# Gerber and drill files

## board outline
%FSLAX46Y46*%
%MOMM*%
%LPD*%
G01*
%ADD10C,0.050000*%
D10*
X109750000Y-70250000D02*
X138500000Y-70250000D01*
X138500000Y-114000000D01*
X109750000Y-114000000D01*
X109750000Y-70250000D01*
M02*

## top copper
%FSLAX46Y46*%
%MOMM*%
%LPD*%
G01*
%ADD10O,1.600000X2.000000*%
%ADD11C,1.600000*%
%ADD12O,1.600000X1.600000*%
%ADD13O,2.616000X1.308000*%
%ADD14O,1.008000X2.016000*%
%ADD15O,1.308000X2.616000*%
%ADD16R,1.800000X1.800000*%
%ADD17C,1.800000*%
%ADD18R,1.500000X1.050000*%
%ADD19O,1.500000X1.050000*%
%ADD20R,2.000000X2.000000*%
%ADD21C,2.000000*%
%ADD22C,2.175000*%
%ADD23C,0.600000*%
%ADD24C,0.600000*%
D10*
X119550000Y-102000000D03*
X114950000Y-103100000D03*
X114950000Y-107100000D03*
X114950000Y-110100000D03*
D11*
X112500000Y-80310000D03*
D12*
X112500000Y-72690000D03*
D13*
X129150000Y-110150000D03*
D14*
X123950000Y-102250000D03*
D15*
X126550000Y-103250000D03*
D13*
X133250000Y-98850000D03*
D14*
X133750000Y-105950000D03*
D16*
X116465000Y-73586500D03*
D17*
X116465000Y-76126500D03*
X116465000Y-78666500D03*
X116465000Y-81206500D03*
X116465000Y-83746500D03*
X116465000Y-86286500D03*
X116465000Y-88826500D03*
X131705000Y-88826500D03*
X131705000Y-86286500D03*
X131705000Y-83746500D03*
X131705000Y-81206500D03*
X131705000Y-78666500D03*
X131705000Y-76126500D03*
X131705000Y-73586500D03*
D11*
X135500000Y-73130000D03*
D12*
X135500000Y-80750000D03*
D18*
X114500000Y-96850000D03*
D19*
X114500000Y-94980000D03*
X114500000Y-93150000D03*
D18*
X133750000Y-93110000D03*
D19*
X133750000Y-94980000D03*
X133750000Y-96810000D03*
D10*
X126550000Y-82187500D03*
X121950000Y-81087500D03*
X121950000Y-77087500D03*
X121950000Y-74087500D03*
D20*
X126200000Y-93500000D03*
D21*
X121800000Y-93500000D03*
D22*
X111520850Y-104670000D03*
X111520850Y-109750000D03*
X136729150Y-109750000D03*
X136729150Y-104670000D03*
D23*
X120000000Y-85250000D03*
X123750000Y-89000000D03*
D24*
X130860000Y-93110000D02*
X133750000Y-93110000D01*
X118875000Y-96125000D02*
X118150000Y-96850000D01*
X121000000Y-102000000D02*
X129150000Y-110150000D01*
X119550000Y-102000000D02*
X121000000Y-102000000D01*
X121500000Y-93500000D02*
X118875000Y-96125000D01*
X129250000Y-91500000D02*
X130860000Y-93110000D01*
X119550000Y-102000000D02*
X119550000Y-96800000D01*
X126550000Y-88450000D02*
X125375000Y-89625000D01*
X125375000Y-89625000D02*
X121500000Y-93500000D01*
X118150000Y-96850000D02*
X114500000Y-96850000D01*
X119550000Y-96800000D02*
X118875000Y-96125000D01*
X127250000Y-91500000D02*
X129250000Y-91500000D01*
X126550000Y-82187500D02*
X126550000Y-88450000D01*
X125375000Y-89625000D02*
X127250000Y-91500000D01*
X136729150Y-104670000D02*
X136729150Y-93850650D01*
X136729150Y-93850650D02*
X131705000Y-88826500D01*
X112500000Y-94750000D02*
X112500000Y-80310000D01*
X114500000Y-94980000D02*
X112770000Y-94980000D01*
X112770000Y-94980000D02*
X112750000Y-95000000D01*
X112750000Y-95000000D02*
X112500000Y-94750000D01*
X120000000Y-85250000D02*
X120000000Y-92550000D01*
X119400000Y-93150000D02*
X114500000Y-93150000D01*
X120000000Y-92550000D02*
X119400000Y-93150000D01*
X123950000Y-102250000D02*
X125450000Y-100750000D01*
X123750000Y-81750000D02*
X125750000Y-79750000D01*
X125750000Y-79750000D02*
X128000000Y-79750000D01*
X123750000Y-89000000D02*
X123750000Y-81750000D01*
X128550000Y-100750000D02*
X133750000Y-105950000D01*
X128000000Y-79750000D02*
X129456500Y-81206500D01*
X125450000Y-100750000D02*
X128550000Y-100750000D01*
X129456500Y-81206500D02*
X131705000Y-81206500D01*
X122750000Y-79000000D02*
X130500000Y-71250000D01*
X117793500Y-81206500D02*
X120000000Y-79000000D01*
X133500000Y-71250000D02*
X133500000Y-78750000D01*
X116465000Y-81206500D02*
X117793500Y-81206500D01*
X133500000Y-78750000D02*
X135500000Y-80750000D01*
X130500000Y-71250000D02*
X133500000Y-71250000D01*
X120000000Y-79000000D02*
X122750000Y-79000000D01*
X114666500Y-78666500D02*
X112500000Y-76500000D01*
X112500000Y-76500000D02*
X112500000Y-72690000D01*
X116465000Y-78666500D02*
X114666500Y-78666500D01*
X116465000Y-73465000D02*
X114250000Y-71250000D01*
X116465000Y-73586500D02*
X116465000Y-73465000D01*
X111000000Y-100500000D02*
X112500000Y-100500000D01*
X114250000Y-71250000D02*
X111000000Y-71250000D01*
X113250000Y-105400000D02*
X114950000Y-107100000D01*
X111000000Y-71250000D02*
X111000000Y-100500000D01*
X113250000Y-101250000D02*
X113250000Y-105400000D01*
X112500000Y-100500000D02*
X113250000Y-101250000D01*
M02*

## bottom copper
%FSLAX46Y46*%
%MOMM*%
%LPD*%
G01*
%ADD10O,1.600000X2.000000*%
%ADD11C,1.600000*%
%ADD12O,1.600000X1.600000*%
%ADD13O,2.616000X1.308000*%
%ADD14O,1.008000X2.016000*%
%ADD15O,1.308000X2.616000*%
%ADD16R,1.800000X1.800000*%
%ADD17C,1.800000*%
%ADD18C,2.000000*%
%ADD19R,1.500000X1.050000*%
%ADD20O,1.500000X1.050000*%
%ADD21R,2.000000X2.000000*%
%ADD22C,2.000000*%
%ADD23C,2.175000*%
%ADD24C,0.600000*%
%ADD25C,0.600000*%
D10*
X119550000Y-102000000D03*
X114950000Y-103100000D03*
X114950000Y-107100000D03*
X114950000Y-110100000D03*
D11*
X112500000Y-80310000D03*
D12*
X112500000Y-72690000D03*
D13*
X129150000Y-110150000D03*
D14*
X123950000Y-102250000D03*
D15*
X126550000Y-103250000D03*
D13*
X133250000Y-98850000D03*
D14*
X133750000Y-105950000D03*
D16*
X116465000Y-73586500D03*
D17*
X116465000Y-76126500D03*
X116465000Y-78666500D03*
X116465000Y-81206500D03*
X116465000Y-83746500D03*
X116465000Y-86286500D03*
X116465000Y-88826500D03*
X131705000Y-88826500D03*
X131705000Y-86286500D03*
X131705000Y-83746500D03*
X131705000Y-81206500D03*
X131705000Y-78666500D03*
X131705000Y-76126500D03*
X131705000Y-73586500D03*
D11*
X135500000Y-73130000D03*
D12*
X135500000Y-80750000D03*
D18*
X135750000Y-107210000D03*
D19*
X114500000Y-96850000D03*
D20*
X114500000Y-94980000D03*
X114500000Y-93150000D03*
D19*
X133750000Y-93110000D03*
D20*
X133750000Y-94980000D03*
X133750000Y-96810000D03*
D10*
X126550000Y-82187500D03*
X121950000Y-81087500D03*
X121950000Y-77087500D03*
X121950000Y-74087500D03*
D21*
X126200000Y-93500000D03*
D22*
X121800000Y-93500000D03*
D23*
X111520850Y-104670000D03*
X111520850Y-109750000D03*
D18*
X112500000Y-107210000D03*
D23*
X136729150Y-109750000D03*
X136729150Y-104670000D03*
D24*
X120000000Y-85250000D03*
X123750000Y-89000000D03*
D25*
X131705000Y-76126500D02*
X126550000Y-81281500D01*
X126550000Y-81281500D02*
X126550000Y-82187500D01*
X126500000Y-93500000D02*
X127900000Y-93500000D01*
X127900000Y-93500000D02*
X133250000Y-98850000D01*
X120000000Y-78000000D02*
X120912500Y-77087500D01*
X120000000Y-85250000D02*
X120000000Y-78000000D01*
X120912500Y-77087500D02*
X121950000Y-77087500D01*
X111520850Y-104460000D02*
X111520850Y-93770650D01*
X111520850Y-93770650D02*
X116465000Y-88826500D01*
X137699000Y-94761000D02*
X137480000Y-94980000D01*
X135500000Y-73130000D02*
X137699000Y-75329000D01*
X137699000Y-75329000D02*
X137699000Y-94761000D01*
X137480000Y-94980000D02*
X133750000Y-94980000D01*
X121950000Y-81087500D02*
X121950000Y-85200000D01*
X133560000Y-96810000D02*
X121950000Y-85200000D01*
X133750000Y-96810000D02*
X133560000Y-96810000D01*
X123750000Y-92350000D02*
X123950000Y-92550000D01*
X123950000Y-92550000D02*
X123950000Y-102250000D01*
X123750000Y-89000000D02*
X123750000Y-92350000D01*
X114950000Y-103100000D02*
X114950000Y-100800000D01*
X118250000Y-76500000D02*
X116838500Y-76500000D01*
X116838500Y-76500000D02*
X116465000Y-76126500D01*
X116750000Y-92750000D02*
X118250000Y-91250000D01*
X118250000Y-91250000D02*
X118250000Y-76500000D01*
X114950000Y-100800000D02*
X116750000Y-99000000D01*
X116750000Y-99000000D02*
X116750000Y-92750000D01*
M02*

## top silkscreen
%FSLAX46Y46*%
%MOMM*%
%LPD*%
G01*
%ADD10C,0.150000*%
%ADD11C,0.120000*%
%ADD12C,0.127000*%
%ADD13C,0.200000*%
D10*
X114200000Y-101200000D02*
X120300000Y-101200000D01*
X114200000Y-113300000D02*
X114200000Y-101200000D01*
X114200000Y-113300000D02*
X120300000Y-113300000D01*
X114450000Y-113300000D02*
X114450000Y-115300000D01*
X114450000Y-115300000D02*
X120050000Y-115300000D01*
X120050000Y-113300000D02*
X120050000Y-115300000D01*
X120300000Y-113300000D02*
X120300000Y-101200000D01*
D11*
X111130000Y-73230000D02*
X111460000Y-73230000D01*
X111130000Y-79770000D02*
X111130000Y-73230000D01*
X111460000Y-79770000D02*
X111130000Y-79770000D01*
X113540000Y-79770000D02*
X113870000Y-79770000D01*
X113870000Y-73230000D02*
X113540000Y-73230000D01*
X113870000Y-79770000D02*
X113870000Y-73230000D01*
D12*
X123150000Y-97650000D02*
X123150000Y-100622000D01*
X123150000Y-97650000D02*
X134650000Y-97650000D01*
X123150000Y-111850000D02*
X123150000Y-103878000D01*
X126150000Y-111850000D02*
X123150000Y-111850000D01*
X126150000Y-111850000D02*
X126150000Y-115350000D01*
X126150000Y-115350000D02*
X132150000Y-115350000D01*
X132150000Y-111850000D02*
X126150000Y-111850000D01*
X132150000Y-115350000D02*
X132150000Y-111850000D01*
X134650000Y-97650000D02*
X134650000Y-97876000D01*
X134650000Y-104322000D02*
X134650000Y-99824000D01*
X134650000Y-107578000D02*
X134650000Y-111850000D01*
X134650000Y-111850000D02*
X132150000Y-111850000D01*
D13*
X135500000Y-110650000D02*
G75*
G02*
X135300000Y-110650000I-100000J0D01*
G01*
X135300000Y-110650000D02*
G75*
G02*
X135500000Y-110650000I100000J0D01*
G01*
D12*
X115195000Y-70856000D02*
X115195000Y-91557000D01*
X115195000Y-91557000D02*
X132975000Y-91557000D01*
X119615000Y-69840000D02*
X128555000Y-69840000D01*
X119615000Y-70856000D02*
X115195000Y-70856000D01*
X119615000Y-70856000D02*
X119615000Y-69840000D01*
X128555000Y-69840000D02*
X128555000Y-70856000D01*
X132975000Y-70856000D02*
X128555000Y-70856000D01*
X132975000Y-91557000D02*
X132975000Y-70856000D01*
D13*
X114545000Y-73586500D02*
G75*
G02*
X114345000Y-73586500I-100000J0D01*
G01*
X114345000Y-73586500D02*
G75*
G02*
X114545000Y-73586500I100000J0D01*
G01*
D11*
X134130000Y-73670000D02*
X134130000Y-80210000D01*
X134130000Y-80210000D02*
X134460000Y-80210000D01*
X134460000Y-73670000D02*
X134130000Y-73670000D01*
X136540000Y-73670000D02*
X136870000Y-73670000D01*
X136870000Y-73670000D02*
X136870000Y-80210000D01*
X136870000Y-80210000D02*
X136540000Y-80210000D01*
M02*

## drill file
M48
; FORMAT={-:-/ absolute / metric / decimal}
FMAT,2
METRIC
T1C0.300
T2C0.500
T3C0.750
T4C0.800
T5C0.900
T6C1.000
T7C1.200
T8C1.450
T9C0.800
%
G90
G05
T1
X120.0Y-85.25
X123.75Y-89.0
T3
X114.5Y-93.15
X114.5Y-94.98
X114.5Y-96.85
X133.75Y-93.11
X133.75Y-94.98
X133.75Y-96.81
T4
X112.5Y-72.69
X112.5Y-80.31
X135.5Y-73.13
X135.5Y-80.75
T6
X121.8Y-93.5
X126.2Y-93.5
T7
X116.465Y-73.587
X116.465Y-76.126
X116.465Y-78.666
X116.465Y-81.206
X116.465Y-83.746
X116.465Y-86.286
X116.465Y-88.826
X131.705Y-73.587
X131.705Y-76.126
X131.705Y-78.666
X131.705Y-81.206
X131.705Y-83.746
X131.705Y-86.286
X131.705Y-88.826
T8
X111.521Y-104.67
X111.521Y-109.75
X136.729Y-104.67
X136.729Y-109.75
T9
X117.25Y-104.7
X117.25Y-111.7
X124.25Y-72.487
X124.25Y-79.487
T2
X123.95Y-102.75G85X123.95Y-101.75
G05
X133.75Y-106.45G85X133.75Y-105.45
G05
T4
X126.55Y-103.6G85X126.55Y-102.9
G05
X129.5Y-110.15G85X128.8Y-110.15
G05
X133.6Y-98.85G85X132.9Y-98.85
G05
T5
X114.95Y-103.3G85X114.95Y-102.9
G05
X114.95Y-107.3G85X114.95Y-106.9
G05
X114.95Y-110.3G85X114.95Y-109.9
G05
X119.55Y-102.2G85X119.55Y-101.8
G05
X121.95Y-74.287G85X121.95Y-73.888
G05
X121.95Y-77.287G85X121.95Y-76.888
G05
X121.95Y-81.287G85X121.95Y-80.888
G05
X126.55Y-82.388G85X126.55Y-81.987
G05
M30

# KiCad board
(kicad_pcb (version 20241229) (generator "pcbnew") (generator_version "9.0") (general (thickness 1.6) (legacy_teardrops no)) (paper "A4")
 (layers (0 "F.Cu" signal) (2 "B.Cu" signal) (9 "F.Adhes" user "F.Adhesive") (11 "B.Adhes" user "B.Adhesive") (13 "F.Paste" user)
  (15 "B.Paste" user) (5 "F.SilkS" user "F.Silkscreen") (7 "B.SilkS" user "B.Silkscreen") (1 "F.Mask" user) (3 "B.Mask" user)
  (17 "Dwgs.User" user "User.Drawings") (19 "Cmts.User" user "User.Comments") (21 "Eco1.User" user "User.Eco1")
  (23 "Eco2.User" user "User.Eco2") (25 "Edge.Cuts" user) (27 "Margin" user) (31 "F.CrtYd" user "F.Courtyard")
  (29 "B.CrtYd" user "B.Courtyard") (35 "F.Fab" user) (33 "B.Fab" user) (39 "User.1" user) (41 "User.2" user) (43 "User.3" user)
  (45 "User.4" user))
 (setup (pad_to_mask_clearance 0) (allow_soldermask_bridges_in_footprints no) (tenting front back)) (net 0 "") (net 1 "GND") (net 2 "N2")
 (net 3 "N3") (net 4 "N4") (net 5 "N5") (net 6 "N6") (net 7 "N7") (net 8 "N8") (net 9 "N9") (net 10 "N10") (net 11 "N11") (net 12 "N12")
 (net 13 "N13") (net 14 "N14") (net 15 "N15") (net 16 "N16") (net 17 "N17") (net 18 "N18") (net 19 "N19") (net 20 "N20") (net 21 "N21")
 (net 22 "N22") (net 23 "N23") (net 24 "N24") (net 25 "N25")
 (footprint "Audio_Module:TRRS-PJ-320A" (layer "F.Cu") (at 117.25 113.3 180)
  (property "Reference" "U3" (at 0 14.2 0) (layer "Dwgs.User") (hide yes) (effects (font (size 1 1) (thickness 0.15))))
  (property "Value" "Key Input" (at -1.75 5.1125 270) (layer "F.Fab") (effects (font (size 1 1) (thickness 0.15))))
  (fp_line (start 3.05 12.1) (end -3.05 12.1) (stroke (width 0.15) (type solid)) (layer "F.SilkS"))
  (fp_line (start 3.05 0) (end 3.05 12.1) (stroke (width 0.15) (type solid)) (layer "F.SilkS"))
  (fp_line (start 3.05 0) (end -3.05 0) (stroke (width 0.15) (type solid)) (layer "F.SilkS"))
  (fp_line (start 2.8 0) (end 2.8 -2) (stroke (width 0.15) (type solid)) (layer "F.SilkS"))
  (fp_line (start 2.8 -2) (end -2.8 -2) (stroke (width 0.15) (type solid)) (layer "F.SilkS"))
  (fp_line (start -2.8 0) (end -2.8 -2) (stroke (width 0.15) (type solid)) (layer "F.SilkS"))
  (fp_line (start -3.05 0) (end -3.05 12.1) (stroke (width 0.15) (type solid)) (layer "F.SilkS"))
  (pad "" np_thru_hole circle (at 0 1.6 180) (size 0.8 0.8) (drill 0.8) (layers "*.Cu" "*.Mask"))
  (pad "" np_thru_hole circle (at 0 8.6 180) (size 0.8 0.8) (drill 0.8) (layers "*.Cu" "*.Mask"))
  (pad "1" thru_hole oval (at -2.3 11.3 180) (size 1.6 2) (drill oval 0.9 1.3) (layers "*.Cu" "*.Mask") (remove_unused_layers no)
   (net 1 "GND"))
  (pad "2" thru_hole oval (at 2.3 10.2 180) (size 1.6 2) (drill oval 0.9 1.3) (layers "*.Cu" "*.Mask") (remove_unused_layers no)
   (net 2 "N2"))
  (pad "3" thru_hole oval (at 2.3 6.2 180) (size 1.6 2) (drill oval 0.9 1.3) (layers "*.Cu" "*.Mask") (remove_unused_layers no) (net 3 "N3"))
  (pad "4" thru_hole oval (at 2.3 3.2 180) (size 1.6 2) (drill oval 0.9 1.3) (layers "*.Cu" "*.Mask") (remove_unused_layers no) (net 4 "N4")))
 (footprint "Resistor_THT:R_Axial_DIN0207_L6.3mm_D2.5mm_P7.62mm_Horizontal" (layer "F.Cu") (at 112.5 80.31 90)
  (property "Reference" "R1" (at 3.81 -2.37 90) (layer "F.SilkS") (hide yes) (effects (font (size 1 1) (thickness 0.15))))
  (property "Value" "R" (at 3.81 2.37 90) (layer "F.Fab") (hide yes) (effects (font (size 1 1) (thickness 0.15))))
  (fp_line (start 7.08 -1.37) (end 7.08 -1.04) (stroke (width 0.12) (type solid)) (layer "F.SilkS"))
  (fp_line (start 0.54 -1.37) (end 7.08 -1.37) (stroke (width 0.12) (type solid)) (layer "F.SilkS"))
  (fp_line (start 0.54 -1.04) (end 0.54 -1.37) (stroke (width 0.12) (type solid)) (layer "F.SilkS"))
  (fp_line (start 0.54 1.04) (end 0.54 1.37) (stroke (width 0.12) (type solid)) (layer "F.SilkS"))
  (fp_line (start 7.08 1.37) (end 7.08 1.04) (stroke (width 0.12) (type solid)) (layer "F.SilkS"))
  (fp_line (start 0.54 1.37) (end 7.08 1.37) (stroke (width 0.12) (type solid)) (layer "F.SilkS"))
  (pad "1" thru_hole circle (at 0 0 90) (size 1.6 1.6) (drill 0.8) (layers "*.Cu" "*.Mask") (remove_unused_layers no) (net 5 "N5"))
  (pad "2" thru_hole oval (at 7.62 0 90) (size 1.6 1.6) (drill 0.8) (layers "*.Cu" "*.Mask") (remove_unused_layers no) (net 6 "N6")))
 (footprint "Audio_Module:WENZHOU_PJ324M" (layer "F.Cu") (at 129.15 104.75 180)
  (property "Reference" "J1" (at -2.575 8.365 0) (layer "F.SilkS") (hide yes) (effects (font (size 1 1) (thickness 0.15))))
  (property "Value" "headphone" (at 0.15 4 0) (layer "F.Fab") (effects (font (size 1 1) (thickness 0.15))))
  (fp_line (start 6 7.1) (end 6 4.128) (stroke (width 0.127) (type solid)) (layer "F.SilkS"))
  (fp_line (start 6 7.1) (end -5.5 7.1) (stroke (width 0.127) (type solid)) (layer "F.SilkS"))
  (fp_line (start 6 -7.1) (end 6 0.872) (stroke (width 0.127) (type solid)) (layer "F.SilkS"))
  (fp_line (start 3 -7.1) (end 6 -7.1) (stroke (width 0.127) (type solid)) (layer "F.SilkS"))
  (fp_line (start 3 -7.1) (end 3 -10.6) (stroke (width 0.127) (type solid)) (layer "F.SilkS"))
  (fp_line (start 3 -10.6) (end -3 -10.6) (stroke (width 0.127) (type solid)) (layer "F.SilkS"))
  (fp_line (start -3 -7.1) (end 3 -7.1) (stroke (width 0.127) (type solid)) (layer "F.SilkS"))
  (fp_line (start -3 -10.6) (end -3 -7.1) (stroke (width 0.127) (type solid)) (layer "F.SilkS"))
  (fp_line (start -5.5 7.1) (end -5.5 6.874) (stroke (width 0.127) (type solid)) (layer "F.SilkS"))
  (fp_line (start -5.5 0.428) (end -5.5 4.926) (stroke (width 0.127) (type solid)) (layer "F.SilkS"))
  (fp_line (start -5.5 -2.828) (end -5.5 -7.1) (stroke (width 0.127) (type solid)) (layer "F.SilkS"))
  (fp_line (start -5.5 -7.1) (end -3 -7.1) (stroke (width 0.127) (type solid)) (layer "F.SilkS"))
  (fp_circle (center -6.25 -5.9) (end -6.15 -5.9) (stroke (width 0.2) (type solid)) (fill no) (layer "F.SilkS"))
  (pad "1" thru_hole oval (at 0 -5.4 180) (size 2.616 1.308) (drill oval 1.5 0.8) (layers "*.Cu" "*.Mask") (remove_unused_layers no)
   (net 1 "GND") (solder_mask_margin 0.102))
  (pad "2" thru_hole oval (at 5.2 2.5 180) (size 1.008 2.016) (drill oval 0.5 1.5) (layers "*.Cu" "*.Mask") (remove_unused_layers no)
   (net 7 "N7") (solder_mask_margin 0.102))
  (pad "3" thru_hole oval (at 2.6 1.5 180) (size 1.308 2.616) (drill oval 0.8 1.5) (layers "*.Cu" "*.Mask") (remove_unused_layers no)
   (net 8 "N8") (solder_mask_margin 0.102))
  (pad "4" thru_hole oval (at -4.1 5.9 180) (size 2.616 1.308) (drill oval 1.5 0.8) (layers "*.Cu" "*.Mask") (remove_unused_layers no)
   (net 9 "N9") (solder_mask_margin 0.102))
  (pad "5" thru_hole oval (at -4.6 -1.2 180) (size 1.008 2.016) (drill oval 0.5 1.5) (layers "*.Cu" "*.Mask") (remove_unused_layers no)
   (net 7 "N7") (solder_mask_margin 0.102)))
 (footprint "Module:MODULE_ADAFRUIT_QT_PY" (layer "F.Cu") (at 124.085 81.2065)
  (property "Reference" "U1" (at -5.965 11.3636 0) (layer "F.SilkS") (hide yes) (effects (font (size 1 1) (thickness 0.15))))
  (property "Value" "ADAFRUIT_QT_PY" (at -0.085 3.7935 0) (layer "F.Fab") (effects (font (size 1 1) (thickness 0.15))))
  (fp_line (start -8.89 -10.3505) (end -8.89 10.3505) (stroke (width 0.127) (type solid)) (layer "F.SilkS"))
  (fp_line (start -8.89 10.3505) (end 8.89 10.3505) (stroke (width 0.127) (type solid)) (layer "F.SilkS"))
  (fp_line (start -4.47 -11.3665) (end 4.47 -11.3665) (stroke (width 0.127) (type solid)) (layer "F.SilkS"))
  (fp_line (start -4.47 -10.3505) (end -8.89 -10.3505) (stroke (width 0.127) (type solid)) (layer "F.SilkS"))
  (fp_line (start -4.47 -10.3505) (end -4.47 -11.3665) (stroke (width 0.127) (type solid)) (layer "F.SilkS"))
  (fp_line (start 4.47 -11.3665) (end 4.47 -10.3505) (stroke (width 0.127) (type solid)) (layer "F.SilkS"))
  (fp_line (start 8.89 -10.3505) (end 4.47 -10.3505) (stroke (width 0.127) (type solid)) (layer "F.SilkS"))
  (fp_line (start 8.89 10.3505) (end 8.89 -10.3505) (stroke (width 0.127) (type solid)) (layer "F.SilkS"))
  (fp_circle (center -9.64 -7.62) (end -9.54 -7.62) (stroke (width 0.2) (type solid)) (fill no) (layer "F.SilkS"))
  (pad "1" thru_hole rect (at -7.62 -7.62) (size 1.8 1.8) (drill 1.2) (layers "*.Cu" "*.Mask") (remove_unused_layers no) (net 3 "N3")
   (solder_mask_margin 0.102))
  (pad "2" thru_hole circle (at -7.62 -5.08) (size 1.8 1.8) (drill 1.2) (layers "*.Cu" "*.Mask") (remove_unused_layers no) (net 2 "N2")
   (solder_mask_margin 0.102))
  (pad "3" thru_hole circle (at -7.62 -2.54) (size 1.8 1.8) (drill 1.2) (layers "*.Cu" "*.Mask") (remove_unused_layers no) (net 6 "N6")
   (solder_mask_margin 0.102))
  (pad "4" thru_hole circle (at -7.62 0) (size 1.8 1.8) (drill 1.2) (layers "*.Cu" "*.Mask") (remove_unused_layers no) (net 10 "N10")
   (solder_mask_margin 0.102))
  (pad "5" thru_hole circle (at -7.62 2.54) (size 1.8 1.8) (drill 1.2) (layers "*.Cu" "*.Mask") (remove_unused_layers no) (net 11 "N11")
   (solder_mask_margin 0.102))
  (pad "6" thru_hole circle (at -7.62 5.08) (size 1.8 1.8) (drill 1.2) (layers "*.Cu" "*.Mask") (remove_unused_layers no) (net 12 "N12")
   (solder_mask_margin 0.102))
  (pad "7" thru_hole circle (at -7.62 7.62) (size 1.8 1.8) (drill 1.2) (layers "*.Cu" "*.Mask") (remove_unused_layers no) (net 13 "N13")
   (solder_mask_margin 0.102))
  (pad "8" thru_hole circle (at 7.62 7.62) (size 1.8 1.8) (drill 1.2) (layers "*.Cu" "*.Mask") (remove_unused_layers no) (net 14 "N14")
   (solder_mask_margin 0.102))
  (pad "9" thru_hole circle (at 7.62 5.08) (size 1.8 1.8) (drill 1.2) (layers "*.Cu" "*.Mask") (remove_unused_layers no) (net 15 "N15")
   (solder_mask_margin 0.102))
  (pad "10" thru_hole circle (at 7.62 2.54) (size 1.8 1.8) (drill 1.2) (layers "*.Cu" "*.Mask") (remove_unused_layers no) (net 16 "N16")
   (solder_mask_margin 0.102))
  (pad "11" thru_hole circle (at 7.62 0) (size 1.8 1.8) (drill 1.2) (layers "*.Cu" "*.Mask") (remove_unused_layers no) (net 7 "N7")
   (solder_mask_margin 0.102))
  (pad "12" thru_hole circle (at 7.62 -2.54) (size 1.8 1.8) (drill 1.2) (layers "*.Cu" "*.Mask") (remove_unused_layers no) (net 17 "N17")
   (solder_mask_margin 0.102))
  (pad "13" thru_hole circle (at 7.62 -5.08) (size 1.8 1.8) (drill 1.2) (layers "*.Cu" "*.Mask") (remove_unused_layers no) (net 1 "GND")
   (solder_mask_margin 0.102))
  (pad "14" thru_hole circle (at 7.62 -7.62) (size 1.8 1.8) (drill 1.2) (layers "*.Cu" "*.Mask") (remove_unused_layers no) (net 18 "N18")
   (solder_mask_margin 0.102)))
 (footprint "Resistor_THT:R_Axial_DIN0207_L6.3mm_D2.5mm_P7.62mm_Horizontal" (layer "F.Cu") (at 135.5 73.13 -90)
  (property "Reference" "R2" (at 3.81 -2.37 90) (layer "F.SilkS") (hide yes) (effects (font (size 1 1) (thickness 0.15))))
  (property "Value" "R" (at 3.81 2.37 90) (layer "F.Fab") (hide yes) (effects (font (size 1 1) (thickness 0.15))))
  (fp_line (start 0.54 1.37) (end 7.08 1.37) (stroke (width 0.12) (type solid)) (layer "F.SilkS"))
  (fp_line (start 7.08 1.37) (end 7.08 1.04) (stroke (width 0.12) (type solid)) (layer "F.SilkS"))
  (fp_line (start 0.54 1.04) (end 0.54 1.37) (stroke (width 0.12) (type solid)) (layer "F.SilkS"))
  (fp_line (start 0.54 -1.04) (end 0.54 -1.37) (stroke (width 0.12) (type solid)) (layer "F.SilkS"))
  (fp_line (start 0.54 -1.37) (end 7.08 -1.37) (stroke (width 0.12) (type solid)) (layer "F.SilkS"))
  (fp_line (start 7.08 -1.37) (end 7.08 -1.04) (stroke (width 0.12) (type solid)) (layer "F.SilkS"))
  (pad "1" thru_hole circle (at 0 0 270) (size 1.6 1.6) (drill 0.8) (layers "*.Cu" "*.Mask") (remove_unused_layers no) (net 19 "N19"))
  (pad "2" thru_hole oval (at 7.62 0 270) (size 1.6 1.6) (drill 0.8) (layers "*.Cu" "*.Mask") (remove_unused_layers no) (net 10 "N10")))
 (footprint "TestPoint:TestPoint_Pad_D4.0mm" (layer "B.Cu") (at 135.75 107.21 180)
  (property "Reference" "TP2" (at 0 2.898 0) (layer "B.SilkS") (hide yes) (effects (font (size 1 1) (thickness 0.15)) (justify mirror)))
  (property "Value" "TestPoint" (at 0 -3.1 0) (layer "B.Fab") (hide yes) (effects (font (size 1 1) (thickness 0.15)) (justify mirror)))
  (pad "1" smd circle (at 0 0 180) (size 2 2) (layers "B.Cu" "B.Mask") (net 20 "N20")))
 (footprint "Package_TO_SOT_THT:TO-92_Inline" (layer "B.Cu") (at 114.5 96.25 90)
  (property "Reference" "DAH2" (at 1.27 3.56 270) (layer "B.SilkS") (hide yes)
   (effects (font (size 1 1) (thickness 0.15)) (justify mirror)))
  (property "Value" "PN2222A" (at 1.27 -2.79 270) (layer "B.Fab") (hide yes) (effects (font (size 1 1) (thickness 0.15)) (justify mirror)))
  (pad "1" thru_hole rect (at -0.6 0 90) (size 1.05 1.5) (drill 0.75) (layers "*.Cu" "*.Mask") (remove_unused_layers no) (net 1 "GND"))
  (pad "2" thru_hole oval (at 1.27 0 90) (size 1.05 1.5) (drill 0.75) (layers "*.Cu" "*.Mask") (remove_unused_layers no) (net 5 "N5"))
  (pad "3" thru_hole oval (at 3.1 0 90) (size 1.05 1.5) (drill 0.75) (layers "*.Cu" "*.Mask") (remove_unused_layers no) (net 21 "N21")))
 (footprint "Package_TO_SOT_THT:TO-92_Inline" (layer "B.Cu") (at 133.75 93.71 -90)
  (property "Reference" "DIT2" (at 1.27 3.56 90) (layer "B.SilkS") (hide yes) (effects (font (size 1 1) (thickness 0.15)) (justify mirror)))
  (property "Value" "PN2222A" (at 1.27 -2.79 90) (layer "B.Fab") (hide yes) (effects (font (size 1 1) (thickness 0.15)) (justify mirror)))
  (pad "1" thru_hole rect (at -0.6 0 270) (size 1.05 1.5) (drill 0.75) (layers "*.Cu" "*.Mask") (remove_unused_layers no) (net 1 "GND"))
  (pad "2" thru_hole oval (at 1.27 0 270) (size 1.05 1.5) (drill 0.75) (layers "*.Cu" "*.Mask") (remove_unused_layers no) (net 19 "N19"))
  (pad "3" thru_hole oval (at 3.1 0 270) (size 1.05 1.5) (drill 0.75) (layers "*.Cu" "*.Mask") (remove_unused_layers no) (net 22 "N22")))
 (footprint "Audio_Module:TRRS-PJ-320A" (layer "B.Cu") (at 124.25 70.8875 180)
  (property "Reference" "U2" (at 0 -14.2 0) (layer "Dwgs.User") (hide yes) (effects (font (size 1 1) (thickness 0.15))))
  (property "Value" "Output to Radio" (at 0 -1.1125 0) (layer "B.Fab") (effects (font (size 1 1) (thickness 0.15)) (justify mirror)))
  (pad "" np_thru_hole circle (at 0 -8.6 180) (size 0.8 0.8) (drill 0.8) (layers "*.Cu" "*.Mask"))
  (pad "" np_thru_hole circle (at 0 -1.6 180) (size 0.8 0.8) (drill 0.8) (layers "*.Cu" "*.Mask"))
  (pad "1" thru_hole oval (at -2.3 -11.3 180) (size 1.6 2) (drill oval 0.9 1.3) (layers "*.Cu" "*.Mask") (remove_unused_layers no)
   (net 1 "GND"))
  (pad "2" thru_hole oval (at 2.3 -10.2 180) (size 1.6 2) (drill oval 0.9 1.3) (layers "*.Cu" "*.Mask") (remove_unused_layers no)
   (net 22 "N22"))
  (pad "3" thru_hole oval (at 2.3 -6.2 180) (size 1.6 2) (drill oval 0.9 1.3) (layers "*.Cu" "*.Mask") (remove_unused_layers no)
   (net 21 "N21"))
  (pad "4" thru_hole oval (at 2.3 -3.2 180) (size 1.6 2) (drill oval 0.9 1.3) (layers "*.Cu" "*.Mask") (remove_unused_layers no)
   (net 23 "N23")))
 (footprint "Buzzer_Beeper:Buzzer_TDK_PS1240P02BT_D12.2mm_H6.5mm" (layer "B.Cu") (at 126.5 93.5 180)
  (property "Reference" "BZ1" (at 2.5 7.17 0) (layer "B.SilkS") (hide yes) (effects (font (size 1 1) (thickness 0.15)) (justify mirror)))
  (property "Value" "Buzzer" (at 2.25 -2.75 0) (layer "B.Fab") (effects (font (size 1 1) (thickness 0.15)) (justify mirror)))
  (pad "1" thru_hole rect (at 0.3 0 180) (size 2 2) (drill 1) (layers "*.Cu" "*.Mask") (remove_unused_layers no) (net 9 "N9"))
  (pad "2" thru_hole circle (at 4.7 0 180) (size 2 2) (drill 1) (layers "*.Cu" "*.Mask") (remove_unused_layers no) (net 1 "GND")))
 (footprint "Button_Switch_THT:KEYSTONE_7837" (layer "B.Cu") (at 111.52085 107.21 -90)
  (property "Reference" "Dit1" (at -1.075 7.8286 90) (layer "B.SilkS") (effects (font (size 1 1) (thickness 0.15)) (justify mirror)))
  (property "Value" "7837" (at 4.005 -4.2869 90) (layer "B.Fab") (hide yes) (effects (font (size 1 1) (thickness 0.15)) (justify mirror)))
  (pad "1_1" thru_hole circle (at -2.54 0 270) (size 2.175 2.175) (drill 1.45) (layers "*.Cu" "*.Mask") (remove_unused_layers no)
   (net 13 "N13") (solder_mask_margin 0.102))
  (pad "1_2" thru_hole circle (at 2.54 0 270) (size 2.175 2.175) (drill 1.45) (layers "*.Cu" "*.Mask") (remove_unused_layers no)
   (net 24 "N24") (solder_mask_margin 0.102)))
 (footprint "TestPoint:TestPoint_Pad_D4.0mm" (layer "B.Cu") (at 112.5 107.21 180)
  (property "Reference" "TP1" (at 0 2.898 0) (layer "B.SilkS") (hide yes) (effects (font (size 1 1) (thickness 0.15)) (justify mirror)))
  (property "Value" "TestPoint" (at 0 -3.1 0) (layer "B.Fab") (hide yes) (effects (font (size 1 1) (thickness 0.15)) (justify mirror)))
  (pad "1" smd circle (at 0 0 180) (size 2 2) (layers "B.Cu" "B.Mask") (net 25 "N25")))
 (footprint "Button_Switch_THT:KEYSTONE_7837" (layer "B.Cu") (at 136.72915 107.21 90)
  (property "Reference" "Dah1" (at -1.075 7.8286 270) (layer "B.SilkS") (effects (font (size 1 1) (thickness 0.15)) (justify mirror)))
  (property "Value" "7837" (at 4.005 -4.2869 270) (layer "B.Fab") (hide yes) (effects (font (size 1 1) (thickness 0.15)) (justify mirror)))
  (pad "1_1" thru_hole circle (at -2.54 0 90) (size 2.175 2.175) (drill 1.45) (layers "*.Cu" "*.Mask") (remove_unused_layers no)
   (solder_mask_margin 0.102))
  (pad "1_2" thru_hole circle (at 2.54 0 90) (size 2.175 2.175) (drill 1.45) (layers "*.Cu" "*.Mask") (remove_unused_layers no)
   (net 14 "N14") (solder_mask_margin 0.102)))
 (gr_rect (start 109.75 70.25) (end 138.5 114) (stroke (width 0.05) (type default)) (fill no) (layer "Edge.Cuts"))
 (segment (start 130.86 93.11) (end 133.75 93.11) (width 0.6) (layer "F.Cu") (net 1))
 (segment (start 118.875 96.125) (end 118.15 96.85) (width 0.6) (layer "F.Cu") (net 1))
 (segment (start 121 102) (end 129.15 110.15) (width 0.6) (layer "F.Cu") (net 1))
 (segment (start 119.55 102) (end 121 102) (width 0.6) (layer "F.Cu") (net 1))
 (segment (start 121.5 93.5) (end 118.875 96.125) (width 0.6) (layer "F.Cu") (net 1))
 (segment (start 129.25 91.5) (end 130.86 93.11) (width 0.6) (layer "F.Cu") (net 1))
 (segment (start 119.55 102) (end 119.55 96.8) (width 0.6) (layer "F.Cu") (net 1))
 (segment (start 126.55 88.45) (end 125.375 89.625) (width 0.6) (layer "F.Cu") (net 1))
 (segment (start 125.375 89.625) (end 121.5 93.5) (width 0.6) (layer "F.Cu") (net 1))
 (segment (start 118.15 96.85) (end 114.5 96.85) (width 0.6) (layer "F.Cu") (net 1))
 (segment (start 119.55 96.8) (end 118.875 96.125) (width 0.6) (layer "F.Cu") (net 1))
 (segment (start 127.25 91.5) (end 129.25 91.5) (width 0.6) (layer "F.Cu") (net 1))
 (segment (start 126.55 82.1875) (end 126.55 88.45) (width 0.6) (layer "F.Cu") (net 1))
 (segment (start 125.375 89.625) (end 127.25 91.5) (width 0.6) (layer "F.Cu") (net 1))
 (segment (start 131.705 76.1265) (end 126.55 81.2815) (width 0.6) (layer "B.Cu") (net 1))
 (segment (start 126.55 81.2815) (end 126.55 82.1875) (width 0.6) (layer "B.Cu") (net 1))
 (segment (start 126.5 93.5) (end 127.9 93.5) (width 0.6) (layer "B.Cu") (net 9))
 (segment (start 127.9 93.5) (end 133.25 98.85) (width 0.6) (layer "B.Cu") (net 9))
 (segment (start 136.72915 104.67) (end 136.72915 93.85065) (width 0.6) (layer "F.Cu") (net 14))
 (segment (start 136.72915 93.85065) (end 131.705 88.8265) (width 0.6) (layer "F.Cu") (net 14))
 (segment (start 112.5 94.75) (end 112.5 80.31) (width 0.6) (layer "F.Cu") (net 5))
 (segment (start 114.5 94.98) (end 112.77 94.98) (width 0.6) (layer "F.Cu") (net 5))
 (segment (start 112.77 94.98) (end 112.75 95) (width 0.6) (layer "F.Cu") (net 5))
 (segment (start 112.75 95) (end 112.5 94.75) (width 0.6) (layer "F.Cu") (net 5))
 (segment (start 120 85.25) (end 120 92.55) (width 0.6) (layer "F.Cu") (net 21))
 (segment (start 119.4 93.15) (end 114.5 93.15) (width 0.6) (layer "F.Cu") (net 21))
 (segment (start 120 92.55) (end 119.4 93.15) (width 0.6) (layer "F.Cu") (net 21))
 (via (at 120 85.25) (size 0.6) (drill 0.3) (layers "F.Cu" "B.Cu") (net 21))
 (segment (start 120 78) (end 120.9125 77.0875) (width 0.6) (layer "B.Cu") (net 21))
 (segment (start 120 85.25) (end 120 78) (width 0.6) (layer "B.Cu") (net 21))
 (segment (start 120.9125 77.0875) (end 121.95 77.0875) (width 0.6) (layer "B.Cu") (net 21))
 (segment (start 111.52085 104.46) (end 111.52085 93.77065) (width 0.6) (layer "B.Cu") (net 13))
 (segment (start 111.52085 93.77065) (end 116.465 88.8265) (width 0.6) (layer "B.Cu") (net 13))
 (segment (start 137.699 94.761) (end 137.48 94.98) (width 0.6) (layer "B.Cu") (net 19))
 (segment (start 135.5 73.13) (end 137.699 75.329) (width 0.6) (layer "B.Cu") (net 19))
 (segment (start 137.699 75.329) (end 137.699 94.761) (width 0.6) (layer "B.Cu") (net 19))
 (segment (start 137.48 94.98) (end 133.75 94.98) (width 0.6) (layer "B.Cu") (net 19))
 (segment (start 121.95 81.0875) (end 121.95 85.2) (width 0.6) (layer "B.Cu") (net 22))
 (segment (start 133.56 96.81) (end 121.95 85.2) (width 0.6) (layer "B.Cu") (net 22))
 (segment (start 133.75 96.81) (end 133.56 96.81) (width 0.6) (layer "B.Cu") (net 22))
 (segment (start 123.95 102.25) (end 125.45 100.75) (width 0.6) (layer "F.Cu") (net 7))
 (segment (start 123.75 81.75) (end 125.75 79.75) (width 0.6) (layer "F.Cu") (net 7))
 (segment (start 125.75 79.75) (end 128 79.75) (width 0.6) (layer "F.Cu") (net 7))
 (segment (start 123.75 89) (end 123.75 81.75) (width 0.6) (layer "F.Cu") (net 7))
 (segment (start 128.55 100.75) (end 133.75 105.95) (width 0.6) (layer "F.Cu") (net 7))
 (segment (start 128 79.75) (end 129.4565 81.2065) (width 0.6) (layer "F.Cu") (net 7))
 (segment (start 125.45 100.75) (end 128.55 100.75) (width 0.6) (layer "F.Cu") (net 7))
 (segment (start 129.4565 81.2065) (end 131.705 81.2065) (width 0.6) (layer "F.Cu") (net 7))
 (via (at 123.75 89) (size 0.6) (drill 0.3) (layers "F.Cu" "B.Cu") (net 7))
 (segment (start 123.75 92.35) (end 123.95 92.55) (width 0.6) (layer "B.Cu") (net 7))
 (segment (start 123.95 92.55) (end 123.95 102.25) (width 0.6) (layer "B.Cu") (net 7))
 (segment (start 123.75 89) (end 123.75 92.35) (width 0.6) (layer "B.Cu") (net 7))
 (segment (start 122.75 79) (end 130.5 71.25) (width 0.6) (layer "F.Cu") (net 10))
 (segment (start 117.7935 81.2065) (end 120 79) (width 0.6) (layer "F.Cu") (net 10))
 (segment (start 133.5 71.25) (end 133.5 78.75) (width 0.6) (layer "F.Cu") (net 10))
 (segment (start 116.465 81.2065) (end 117.7935 81.2065) (width 0.6) (layer "F.Cu") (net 10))
 (segment (start 133.5 78.75) (end 135.5 80.75) (width 0.6) (layer "F.Cu") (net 10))
 (segment (start 130.5 71.25) (end 133.5 71.25) (width 0.6) (layer "F.Cu") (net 10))
 (segment (start 120 79) (end 122.75 79) (width 0.6) (layer "F.Cu") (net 10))
 (segment (start 114.6665 78.6665) (end 112.5 76.5) (width 0.6) (layer "F.Cu") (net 6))
 (segment (start 112.5 76.5) (end 112.5 72.69) (width 0.6) (layer "F.Cu") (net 6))
 (segment (start 116.465 78.6665) (end 114.6665 78.6665) (width 0.6) (layer "F.Cu") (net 6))
 (segment (start 114.95 103.1) (end 114.95 100.8) (width 0.6) (layer "B.Cu") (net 2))
 (segment (start 118.25 76.5) (end 116.8385 76.5) (width 0.6) (layer "B.Cu") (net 2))
 (segment (start 116.8385 76.5) (end 116.465 76.1265) (width 0.6) (layer "B.Cu") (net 2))
 (segment (start 116.75 92.75) (end 118.25 91.25) (width 0.6) (layer "B.Cu") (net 2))
 (segment (start 118.25 91.25) (end 118.25 76.5) (width 0.6) (layer "B.Cu") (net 2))
 (segment (start 114.95 100.8) (end 116.75 99) (width 0.6) (layer "B.Cu") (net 2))
 (segment (start 116.75 99) (end 116.75 92.75) (width 0.6) (layer "B.Cu") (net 2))
 (segment (start 116.465 73.465) (end 114.25 71.25) (width 0.6) (layer "F.Cu") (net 3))
 (segment (start 116.465 73.5865) (end 116.465 73.465) (width 0.6) (layer "F.Cu") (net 3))
 (segment (start 111 100.5) (end 112.5 100.5) (width 0.6) (layer "F.Cu") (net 3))
 (segment (start 114.25 71.25) (end 111 71.25) (width 0.6) (layer "F.Cu") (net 3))
 (segment (start 113.25 105.4) (end 114.95 107.1) (width 0.6) (layer "F.Cu") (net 3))
 (segment (start 111 71.25) (end 111 100.5) (width 0.6) (layer "F.Cu") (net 3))
 (segment (start 113.25 101.25) (end 113.25 105.4) (width 0.6) (layer "F.Cu") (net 3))
 (segment (start 112.5 100.5) (end 113.25 101.25) (width 0.6) (layer "F.Cu") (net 3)))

